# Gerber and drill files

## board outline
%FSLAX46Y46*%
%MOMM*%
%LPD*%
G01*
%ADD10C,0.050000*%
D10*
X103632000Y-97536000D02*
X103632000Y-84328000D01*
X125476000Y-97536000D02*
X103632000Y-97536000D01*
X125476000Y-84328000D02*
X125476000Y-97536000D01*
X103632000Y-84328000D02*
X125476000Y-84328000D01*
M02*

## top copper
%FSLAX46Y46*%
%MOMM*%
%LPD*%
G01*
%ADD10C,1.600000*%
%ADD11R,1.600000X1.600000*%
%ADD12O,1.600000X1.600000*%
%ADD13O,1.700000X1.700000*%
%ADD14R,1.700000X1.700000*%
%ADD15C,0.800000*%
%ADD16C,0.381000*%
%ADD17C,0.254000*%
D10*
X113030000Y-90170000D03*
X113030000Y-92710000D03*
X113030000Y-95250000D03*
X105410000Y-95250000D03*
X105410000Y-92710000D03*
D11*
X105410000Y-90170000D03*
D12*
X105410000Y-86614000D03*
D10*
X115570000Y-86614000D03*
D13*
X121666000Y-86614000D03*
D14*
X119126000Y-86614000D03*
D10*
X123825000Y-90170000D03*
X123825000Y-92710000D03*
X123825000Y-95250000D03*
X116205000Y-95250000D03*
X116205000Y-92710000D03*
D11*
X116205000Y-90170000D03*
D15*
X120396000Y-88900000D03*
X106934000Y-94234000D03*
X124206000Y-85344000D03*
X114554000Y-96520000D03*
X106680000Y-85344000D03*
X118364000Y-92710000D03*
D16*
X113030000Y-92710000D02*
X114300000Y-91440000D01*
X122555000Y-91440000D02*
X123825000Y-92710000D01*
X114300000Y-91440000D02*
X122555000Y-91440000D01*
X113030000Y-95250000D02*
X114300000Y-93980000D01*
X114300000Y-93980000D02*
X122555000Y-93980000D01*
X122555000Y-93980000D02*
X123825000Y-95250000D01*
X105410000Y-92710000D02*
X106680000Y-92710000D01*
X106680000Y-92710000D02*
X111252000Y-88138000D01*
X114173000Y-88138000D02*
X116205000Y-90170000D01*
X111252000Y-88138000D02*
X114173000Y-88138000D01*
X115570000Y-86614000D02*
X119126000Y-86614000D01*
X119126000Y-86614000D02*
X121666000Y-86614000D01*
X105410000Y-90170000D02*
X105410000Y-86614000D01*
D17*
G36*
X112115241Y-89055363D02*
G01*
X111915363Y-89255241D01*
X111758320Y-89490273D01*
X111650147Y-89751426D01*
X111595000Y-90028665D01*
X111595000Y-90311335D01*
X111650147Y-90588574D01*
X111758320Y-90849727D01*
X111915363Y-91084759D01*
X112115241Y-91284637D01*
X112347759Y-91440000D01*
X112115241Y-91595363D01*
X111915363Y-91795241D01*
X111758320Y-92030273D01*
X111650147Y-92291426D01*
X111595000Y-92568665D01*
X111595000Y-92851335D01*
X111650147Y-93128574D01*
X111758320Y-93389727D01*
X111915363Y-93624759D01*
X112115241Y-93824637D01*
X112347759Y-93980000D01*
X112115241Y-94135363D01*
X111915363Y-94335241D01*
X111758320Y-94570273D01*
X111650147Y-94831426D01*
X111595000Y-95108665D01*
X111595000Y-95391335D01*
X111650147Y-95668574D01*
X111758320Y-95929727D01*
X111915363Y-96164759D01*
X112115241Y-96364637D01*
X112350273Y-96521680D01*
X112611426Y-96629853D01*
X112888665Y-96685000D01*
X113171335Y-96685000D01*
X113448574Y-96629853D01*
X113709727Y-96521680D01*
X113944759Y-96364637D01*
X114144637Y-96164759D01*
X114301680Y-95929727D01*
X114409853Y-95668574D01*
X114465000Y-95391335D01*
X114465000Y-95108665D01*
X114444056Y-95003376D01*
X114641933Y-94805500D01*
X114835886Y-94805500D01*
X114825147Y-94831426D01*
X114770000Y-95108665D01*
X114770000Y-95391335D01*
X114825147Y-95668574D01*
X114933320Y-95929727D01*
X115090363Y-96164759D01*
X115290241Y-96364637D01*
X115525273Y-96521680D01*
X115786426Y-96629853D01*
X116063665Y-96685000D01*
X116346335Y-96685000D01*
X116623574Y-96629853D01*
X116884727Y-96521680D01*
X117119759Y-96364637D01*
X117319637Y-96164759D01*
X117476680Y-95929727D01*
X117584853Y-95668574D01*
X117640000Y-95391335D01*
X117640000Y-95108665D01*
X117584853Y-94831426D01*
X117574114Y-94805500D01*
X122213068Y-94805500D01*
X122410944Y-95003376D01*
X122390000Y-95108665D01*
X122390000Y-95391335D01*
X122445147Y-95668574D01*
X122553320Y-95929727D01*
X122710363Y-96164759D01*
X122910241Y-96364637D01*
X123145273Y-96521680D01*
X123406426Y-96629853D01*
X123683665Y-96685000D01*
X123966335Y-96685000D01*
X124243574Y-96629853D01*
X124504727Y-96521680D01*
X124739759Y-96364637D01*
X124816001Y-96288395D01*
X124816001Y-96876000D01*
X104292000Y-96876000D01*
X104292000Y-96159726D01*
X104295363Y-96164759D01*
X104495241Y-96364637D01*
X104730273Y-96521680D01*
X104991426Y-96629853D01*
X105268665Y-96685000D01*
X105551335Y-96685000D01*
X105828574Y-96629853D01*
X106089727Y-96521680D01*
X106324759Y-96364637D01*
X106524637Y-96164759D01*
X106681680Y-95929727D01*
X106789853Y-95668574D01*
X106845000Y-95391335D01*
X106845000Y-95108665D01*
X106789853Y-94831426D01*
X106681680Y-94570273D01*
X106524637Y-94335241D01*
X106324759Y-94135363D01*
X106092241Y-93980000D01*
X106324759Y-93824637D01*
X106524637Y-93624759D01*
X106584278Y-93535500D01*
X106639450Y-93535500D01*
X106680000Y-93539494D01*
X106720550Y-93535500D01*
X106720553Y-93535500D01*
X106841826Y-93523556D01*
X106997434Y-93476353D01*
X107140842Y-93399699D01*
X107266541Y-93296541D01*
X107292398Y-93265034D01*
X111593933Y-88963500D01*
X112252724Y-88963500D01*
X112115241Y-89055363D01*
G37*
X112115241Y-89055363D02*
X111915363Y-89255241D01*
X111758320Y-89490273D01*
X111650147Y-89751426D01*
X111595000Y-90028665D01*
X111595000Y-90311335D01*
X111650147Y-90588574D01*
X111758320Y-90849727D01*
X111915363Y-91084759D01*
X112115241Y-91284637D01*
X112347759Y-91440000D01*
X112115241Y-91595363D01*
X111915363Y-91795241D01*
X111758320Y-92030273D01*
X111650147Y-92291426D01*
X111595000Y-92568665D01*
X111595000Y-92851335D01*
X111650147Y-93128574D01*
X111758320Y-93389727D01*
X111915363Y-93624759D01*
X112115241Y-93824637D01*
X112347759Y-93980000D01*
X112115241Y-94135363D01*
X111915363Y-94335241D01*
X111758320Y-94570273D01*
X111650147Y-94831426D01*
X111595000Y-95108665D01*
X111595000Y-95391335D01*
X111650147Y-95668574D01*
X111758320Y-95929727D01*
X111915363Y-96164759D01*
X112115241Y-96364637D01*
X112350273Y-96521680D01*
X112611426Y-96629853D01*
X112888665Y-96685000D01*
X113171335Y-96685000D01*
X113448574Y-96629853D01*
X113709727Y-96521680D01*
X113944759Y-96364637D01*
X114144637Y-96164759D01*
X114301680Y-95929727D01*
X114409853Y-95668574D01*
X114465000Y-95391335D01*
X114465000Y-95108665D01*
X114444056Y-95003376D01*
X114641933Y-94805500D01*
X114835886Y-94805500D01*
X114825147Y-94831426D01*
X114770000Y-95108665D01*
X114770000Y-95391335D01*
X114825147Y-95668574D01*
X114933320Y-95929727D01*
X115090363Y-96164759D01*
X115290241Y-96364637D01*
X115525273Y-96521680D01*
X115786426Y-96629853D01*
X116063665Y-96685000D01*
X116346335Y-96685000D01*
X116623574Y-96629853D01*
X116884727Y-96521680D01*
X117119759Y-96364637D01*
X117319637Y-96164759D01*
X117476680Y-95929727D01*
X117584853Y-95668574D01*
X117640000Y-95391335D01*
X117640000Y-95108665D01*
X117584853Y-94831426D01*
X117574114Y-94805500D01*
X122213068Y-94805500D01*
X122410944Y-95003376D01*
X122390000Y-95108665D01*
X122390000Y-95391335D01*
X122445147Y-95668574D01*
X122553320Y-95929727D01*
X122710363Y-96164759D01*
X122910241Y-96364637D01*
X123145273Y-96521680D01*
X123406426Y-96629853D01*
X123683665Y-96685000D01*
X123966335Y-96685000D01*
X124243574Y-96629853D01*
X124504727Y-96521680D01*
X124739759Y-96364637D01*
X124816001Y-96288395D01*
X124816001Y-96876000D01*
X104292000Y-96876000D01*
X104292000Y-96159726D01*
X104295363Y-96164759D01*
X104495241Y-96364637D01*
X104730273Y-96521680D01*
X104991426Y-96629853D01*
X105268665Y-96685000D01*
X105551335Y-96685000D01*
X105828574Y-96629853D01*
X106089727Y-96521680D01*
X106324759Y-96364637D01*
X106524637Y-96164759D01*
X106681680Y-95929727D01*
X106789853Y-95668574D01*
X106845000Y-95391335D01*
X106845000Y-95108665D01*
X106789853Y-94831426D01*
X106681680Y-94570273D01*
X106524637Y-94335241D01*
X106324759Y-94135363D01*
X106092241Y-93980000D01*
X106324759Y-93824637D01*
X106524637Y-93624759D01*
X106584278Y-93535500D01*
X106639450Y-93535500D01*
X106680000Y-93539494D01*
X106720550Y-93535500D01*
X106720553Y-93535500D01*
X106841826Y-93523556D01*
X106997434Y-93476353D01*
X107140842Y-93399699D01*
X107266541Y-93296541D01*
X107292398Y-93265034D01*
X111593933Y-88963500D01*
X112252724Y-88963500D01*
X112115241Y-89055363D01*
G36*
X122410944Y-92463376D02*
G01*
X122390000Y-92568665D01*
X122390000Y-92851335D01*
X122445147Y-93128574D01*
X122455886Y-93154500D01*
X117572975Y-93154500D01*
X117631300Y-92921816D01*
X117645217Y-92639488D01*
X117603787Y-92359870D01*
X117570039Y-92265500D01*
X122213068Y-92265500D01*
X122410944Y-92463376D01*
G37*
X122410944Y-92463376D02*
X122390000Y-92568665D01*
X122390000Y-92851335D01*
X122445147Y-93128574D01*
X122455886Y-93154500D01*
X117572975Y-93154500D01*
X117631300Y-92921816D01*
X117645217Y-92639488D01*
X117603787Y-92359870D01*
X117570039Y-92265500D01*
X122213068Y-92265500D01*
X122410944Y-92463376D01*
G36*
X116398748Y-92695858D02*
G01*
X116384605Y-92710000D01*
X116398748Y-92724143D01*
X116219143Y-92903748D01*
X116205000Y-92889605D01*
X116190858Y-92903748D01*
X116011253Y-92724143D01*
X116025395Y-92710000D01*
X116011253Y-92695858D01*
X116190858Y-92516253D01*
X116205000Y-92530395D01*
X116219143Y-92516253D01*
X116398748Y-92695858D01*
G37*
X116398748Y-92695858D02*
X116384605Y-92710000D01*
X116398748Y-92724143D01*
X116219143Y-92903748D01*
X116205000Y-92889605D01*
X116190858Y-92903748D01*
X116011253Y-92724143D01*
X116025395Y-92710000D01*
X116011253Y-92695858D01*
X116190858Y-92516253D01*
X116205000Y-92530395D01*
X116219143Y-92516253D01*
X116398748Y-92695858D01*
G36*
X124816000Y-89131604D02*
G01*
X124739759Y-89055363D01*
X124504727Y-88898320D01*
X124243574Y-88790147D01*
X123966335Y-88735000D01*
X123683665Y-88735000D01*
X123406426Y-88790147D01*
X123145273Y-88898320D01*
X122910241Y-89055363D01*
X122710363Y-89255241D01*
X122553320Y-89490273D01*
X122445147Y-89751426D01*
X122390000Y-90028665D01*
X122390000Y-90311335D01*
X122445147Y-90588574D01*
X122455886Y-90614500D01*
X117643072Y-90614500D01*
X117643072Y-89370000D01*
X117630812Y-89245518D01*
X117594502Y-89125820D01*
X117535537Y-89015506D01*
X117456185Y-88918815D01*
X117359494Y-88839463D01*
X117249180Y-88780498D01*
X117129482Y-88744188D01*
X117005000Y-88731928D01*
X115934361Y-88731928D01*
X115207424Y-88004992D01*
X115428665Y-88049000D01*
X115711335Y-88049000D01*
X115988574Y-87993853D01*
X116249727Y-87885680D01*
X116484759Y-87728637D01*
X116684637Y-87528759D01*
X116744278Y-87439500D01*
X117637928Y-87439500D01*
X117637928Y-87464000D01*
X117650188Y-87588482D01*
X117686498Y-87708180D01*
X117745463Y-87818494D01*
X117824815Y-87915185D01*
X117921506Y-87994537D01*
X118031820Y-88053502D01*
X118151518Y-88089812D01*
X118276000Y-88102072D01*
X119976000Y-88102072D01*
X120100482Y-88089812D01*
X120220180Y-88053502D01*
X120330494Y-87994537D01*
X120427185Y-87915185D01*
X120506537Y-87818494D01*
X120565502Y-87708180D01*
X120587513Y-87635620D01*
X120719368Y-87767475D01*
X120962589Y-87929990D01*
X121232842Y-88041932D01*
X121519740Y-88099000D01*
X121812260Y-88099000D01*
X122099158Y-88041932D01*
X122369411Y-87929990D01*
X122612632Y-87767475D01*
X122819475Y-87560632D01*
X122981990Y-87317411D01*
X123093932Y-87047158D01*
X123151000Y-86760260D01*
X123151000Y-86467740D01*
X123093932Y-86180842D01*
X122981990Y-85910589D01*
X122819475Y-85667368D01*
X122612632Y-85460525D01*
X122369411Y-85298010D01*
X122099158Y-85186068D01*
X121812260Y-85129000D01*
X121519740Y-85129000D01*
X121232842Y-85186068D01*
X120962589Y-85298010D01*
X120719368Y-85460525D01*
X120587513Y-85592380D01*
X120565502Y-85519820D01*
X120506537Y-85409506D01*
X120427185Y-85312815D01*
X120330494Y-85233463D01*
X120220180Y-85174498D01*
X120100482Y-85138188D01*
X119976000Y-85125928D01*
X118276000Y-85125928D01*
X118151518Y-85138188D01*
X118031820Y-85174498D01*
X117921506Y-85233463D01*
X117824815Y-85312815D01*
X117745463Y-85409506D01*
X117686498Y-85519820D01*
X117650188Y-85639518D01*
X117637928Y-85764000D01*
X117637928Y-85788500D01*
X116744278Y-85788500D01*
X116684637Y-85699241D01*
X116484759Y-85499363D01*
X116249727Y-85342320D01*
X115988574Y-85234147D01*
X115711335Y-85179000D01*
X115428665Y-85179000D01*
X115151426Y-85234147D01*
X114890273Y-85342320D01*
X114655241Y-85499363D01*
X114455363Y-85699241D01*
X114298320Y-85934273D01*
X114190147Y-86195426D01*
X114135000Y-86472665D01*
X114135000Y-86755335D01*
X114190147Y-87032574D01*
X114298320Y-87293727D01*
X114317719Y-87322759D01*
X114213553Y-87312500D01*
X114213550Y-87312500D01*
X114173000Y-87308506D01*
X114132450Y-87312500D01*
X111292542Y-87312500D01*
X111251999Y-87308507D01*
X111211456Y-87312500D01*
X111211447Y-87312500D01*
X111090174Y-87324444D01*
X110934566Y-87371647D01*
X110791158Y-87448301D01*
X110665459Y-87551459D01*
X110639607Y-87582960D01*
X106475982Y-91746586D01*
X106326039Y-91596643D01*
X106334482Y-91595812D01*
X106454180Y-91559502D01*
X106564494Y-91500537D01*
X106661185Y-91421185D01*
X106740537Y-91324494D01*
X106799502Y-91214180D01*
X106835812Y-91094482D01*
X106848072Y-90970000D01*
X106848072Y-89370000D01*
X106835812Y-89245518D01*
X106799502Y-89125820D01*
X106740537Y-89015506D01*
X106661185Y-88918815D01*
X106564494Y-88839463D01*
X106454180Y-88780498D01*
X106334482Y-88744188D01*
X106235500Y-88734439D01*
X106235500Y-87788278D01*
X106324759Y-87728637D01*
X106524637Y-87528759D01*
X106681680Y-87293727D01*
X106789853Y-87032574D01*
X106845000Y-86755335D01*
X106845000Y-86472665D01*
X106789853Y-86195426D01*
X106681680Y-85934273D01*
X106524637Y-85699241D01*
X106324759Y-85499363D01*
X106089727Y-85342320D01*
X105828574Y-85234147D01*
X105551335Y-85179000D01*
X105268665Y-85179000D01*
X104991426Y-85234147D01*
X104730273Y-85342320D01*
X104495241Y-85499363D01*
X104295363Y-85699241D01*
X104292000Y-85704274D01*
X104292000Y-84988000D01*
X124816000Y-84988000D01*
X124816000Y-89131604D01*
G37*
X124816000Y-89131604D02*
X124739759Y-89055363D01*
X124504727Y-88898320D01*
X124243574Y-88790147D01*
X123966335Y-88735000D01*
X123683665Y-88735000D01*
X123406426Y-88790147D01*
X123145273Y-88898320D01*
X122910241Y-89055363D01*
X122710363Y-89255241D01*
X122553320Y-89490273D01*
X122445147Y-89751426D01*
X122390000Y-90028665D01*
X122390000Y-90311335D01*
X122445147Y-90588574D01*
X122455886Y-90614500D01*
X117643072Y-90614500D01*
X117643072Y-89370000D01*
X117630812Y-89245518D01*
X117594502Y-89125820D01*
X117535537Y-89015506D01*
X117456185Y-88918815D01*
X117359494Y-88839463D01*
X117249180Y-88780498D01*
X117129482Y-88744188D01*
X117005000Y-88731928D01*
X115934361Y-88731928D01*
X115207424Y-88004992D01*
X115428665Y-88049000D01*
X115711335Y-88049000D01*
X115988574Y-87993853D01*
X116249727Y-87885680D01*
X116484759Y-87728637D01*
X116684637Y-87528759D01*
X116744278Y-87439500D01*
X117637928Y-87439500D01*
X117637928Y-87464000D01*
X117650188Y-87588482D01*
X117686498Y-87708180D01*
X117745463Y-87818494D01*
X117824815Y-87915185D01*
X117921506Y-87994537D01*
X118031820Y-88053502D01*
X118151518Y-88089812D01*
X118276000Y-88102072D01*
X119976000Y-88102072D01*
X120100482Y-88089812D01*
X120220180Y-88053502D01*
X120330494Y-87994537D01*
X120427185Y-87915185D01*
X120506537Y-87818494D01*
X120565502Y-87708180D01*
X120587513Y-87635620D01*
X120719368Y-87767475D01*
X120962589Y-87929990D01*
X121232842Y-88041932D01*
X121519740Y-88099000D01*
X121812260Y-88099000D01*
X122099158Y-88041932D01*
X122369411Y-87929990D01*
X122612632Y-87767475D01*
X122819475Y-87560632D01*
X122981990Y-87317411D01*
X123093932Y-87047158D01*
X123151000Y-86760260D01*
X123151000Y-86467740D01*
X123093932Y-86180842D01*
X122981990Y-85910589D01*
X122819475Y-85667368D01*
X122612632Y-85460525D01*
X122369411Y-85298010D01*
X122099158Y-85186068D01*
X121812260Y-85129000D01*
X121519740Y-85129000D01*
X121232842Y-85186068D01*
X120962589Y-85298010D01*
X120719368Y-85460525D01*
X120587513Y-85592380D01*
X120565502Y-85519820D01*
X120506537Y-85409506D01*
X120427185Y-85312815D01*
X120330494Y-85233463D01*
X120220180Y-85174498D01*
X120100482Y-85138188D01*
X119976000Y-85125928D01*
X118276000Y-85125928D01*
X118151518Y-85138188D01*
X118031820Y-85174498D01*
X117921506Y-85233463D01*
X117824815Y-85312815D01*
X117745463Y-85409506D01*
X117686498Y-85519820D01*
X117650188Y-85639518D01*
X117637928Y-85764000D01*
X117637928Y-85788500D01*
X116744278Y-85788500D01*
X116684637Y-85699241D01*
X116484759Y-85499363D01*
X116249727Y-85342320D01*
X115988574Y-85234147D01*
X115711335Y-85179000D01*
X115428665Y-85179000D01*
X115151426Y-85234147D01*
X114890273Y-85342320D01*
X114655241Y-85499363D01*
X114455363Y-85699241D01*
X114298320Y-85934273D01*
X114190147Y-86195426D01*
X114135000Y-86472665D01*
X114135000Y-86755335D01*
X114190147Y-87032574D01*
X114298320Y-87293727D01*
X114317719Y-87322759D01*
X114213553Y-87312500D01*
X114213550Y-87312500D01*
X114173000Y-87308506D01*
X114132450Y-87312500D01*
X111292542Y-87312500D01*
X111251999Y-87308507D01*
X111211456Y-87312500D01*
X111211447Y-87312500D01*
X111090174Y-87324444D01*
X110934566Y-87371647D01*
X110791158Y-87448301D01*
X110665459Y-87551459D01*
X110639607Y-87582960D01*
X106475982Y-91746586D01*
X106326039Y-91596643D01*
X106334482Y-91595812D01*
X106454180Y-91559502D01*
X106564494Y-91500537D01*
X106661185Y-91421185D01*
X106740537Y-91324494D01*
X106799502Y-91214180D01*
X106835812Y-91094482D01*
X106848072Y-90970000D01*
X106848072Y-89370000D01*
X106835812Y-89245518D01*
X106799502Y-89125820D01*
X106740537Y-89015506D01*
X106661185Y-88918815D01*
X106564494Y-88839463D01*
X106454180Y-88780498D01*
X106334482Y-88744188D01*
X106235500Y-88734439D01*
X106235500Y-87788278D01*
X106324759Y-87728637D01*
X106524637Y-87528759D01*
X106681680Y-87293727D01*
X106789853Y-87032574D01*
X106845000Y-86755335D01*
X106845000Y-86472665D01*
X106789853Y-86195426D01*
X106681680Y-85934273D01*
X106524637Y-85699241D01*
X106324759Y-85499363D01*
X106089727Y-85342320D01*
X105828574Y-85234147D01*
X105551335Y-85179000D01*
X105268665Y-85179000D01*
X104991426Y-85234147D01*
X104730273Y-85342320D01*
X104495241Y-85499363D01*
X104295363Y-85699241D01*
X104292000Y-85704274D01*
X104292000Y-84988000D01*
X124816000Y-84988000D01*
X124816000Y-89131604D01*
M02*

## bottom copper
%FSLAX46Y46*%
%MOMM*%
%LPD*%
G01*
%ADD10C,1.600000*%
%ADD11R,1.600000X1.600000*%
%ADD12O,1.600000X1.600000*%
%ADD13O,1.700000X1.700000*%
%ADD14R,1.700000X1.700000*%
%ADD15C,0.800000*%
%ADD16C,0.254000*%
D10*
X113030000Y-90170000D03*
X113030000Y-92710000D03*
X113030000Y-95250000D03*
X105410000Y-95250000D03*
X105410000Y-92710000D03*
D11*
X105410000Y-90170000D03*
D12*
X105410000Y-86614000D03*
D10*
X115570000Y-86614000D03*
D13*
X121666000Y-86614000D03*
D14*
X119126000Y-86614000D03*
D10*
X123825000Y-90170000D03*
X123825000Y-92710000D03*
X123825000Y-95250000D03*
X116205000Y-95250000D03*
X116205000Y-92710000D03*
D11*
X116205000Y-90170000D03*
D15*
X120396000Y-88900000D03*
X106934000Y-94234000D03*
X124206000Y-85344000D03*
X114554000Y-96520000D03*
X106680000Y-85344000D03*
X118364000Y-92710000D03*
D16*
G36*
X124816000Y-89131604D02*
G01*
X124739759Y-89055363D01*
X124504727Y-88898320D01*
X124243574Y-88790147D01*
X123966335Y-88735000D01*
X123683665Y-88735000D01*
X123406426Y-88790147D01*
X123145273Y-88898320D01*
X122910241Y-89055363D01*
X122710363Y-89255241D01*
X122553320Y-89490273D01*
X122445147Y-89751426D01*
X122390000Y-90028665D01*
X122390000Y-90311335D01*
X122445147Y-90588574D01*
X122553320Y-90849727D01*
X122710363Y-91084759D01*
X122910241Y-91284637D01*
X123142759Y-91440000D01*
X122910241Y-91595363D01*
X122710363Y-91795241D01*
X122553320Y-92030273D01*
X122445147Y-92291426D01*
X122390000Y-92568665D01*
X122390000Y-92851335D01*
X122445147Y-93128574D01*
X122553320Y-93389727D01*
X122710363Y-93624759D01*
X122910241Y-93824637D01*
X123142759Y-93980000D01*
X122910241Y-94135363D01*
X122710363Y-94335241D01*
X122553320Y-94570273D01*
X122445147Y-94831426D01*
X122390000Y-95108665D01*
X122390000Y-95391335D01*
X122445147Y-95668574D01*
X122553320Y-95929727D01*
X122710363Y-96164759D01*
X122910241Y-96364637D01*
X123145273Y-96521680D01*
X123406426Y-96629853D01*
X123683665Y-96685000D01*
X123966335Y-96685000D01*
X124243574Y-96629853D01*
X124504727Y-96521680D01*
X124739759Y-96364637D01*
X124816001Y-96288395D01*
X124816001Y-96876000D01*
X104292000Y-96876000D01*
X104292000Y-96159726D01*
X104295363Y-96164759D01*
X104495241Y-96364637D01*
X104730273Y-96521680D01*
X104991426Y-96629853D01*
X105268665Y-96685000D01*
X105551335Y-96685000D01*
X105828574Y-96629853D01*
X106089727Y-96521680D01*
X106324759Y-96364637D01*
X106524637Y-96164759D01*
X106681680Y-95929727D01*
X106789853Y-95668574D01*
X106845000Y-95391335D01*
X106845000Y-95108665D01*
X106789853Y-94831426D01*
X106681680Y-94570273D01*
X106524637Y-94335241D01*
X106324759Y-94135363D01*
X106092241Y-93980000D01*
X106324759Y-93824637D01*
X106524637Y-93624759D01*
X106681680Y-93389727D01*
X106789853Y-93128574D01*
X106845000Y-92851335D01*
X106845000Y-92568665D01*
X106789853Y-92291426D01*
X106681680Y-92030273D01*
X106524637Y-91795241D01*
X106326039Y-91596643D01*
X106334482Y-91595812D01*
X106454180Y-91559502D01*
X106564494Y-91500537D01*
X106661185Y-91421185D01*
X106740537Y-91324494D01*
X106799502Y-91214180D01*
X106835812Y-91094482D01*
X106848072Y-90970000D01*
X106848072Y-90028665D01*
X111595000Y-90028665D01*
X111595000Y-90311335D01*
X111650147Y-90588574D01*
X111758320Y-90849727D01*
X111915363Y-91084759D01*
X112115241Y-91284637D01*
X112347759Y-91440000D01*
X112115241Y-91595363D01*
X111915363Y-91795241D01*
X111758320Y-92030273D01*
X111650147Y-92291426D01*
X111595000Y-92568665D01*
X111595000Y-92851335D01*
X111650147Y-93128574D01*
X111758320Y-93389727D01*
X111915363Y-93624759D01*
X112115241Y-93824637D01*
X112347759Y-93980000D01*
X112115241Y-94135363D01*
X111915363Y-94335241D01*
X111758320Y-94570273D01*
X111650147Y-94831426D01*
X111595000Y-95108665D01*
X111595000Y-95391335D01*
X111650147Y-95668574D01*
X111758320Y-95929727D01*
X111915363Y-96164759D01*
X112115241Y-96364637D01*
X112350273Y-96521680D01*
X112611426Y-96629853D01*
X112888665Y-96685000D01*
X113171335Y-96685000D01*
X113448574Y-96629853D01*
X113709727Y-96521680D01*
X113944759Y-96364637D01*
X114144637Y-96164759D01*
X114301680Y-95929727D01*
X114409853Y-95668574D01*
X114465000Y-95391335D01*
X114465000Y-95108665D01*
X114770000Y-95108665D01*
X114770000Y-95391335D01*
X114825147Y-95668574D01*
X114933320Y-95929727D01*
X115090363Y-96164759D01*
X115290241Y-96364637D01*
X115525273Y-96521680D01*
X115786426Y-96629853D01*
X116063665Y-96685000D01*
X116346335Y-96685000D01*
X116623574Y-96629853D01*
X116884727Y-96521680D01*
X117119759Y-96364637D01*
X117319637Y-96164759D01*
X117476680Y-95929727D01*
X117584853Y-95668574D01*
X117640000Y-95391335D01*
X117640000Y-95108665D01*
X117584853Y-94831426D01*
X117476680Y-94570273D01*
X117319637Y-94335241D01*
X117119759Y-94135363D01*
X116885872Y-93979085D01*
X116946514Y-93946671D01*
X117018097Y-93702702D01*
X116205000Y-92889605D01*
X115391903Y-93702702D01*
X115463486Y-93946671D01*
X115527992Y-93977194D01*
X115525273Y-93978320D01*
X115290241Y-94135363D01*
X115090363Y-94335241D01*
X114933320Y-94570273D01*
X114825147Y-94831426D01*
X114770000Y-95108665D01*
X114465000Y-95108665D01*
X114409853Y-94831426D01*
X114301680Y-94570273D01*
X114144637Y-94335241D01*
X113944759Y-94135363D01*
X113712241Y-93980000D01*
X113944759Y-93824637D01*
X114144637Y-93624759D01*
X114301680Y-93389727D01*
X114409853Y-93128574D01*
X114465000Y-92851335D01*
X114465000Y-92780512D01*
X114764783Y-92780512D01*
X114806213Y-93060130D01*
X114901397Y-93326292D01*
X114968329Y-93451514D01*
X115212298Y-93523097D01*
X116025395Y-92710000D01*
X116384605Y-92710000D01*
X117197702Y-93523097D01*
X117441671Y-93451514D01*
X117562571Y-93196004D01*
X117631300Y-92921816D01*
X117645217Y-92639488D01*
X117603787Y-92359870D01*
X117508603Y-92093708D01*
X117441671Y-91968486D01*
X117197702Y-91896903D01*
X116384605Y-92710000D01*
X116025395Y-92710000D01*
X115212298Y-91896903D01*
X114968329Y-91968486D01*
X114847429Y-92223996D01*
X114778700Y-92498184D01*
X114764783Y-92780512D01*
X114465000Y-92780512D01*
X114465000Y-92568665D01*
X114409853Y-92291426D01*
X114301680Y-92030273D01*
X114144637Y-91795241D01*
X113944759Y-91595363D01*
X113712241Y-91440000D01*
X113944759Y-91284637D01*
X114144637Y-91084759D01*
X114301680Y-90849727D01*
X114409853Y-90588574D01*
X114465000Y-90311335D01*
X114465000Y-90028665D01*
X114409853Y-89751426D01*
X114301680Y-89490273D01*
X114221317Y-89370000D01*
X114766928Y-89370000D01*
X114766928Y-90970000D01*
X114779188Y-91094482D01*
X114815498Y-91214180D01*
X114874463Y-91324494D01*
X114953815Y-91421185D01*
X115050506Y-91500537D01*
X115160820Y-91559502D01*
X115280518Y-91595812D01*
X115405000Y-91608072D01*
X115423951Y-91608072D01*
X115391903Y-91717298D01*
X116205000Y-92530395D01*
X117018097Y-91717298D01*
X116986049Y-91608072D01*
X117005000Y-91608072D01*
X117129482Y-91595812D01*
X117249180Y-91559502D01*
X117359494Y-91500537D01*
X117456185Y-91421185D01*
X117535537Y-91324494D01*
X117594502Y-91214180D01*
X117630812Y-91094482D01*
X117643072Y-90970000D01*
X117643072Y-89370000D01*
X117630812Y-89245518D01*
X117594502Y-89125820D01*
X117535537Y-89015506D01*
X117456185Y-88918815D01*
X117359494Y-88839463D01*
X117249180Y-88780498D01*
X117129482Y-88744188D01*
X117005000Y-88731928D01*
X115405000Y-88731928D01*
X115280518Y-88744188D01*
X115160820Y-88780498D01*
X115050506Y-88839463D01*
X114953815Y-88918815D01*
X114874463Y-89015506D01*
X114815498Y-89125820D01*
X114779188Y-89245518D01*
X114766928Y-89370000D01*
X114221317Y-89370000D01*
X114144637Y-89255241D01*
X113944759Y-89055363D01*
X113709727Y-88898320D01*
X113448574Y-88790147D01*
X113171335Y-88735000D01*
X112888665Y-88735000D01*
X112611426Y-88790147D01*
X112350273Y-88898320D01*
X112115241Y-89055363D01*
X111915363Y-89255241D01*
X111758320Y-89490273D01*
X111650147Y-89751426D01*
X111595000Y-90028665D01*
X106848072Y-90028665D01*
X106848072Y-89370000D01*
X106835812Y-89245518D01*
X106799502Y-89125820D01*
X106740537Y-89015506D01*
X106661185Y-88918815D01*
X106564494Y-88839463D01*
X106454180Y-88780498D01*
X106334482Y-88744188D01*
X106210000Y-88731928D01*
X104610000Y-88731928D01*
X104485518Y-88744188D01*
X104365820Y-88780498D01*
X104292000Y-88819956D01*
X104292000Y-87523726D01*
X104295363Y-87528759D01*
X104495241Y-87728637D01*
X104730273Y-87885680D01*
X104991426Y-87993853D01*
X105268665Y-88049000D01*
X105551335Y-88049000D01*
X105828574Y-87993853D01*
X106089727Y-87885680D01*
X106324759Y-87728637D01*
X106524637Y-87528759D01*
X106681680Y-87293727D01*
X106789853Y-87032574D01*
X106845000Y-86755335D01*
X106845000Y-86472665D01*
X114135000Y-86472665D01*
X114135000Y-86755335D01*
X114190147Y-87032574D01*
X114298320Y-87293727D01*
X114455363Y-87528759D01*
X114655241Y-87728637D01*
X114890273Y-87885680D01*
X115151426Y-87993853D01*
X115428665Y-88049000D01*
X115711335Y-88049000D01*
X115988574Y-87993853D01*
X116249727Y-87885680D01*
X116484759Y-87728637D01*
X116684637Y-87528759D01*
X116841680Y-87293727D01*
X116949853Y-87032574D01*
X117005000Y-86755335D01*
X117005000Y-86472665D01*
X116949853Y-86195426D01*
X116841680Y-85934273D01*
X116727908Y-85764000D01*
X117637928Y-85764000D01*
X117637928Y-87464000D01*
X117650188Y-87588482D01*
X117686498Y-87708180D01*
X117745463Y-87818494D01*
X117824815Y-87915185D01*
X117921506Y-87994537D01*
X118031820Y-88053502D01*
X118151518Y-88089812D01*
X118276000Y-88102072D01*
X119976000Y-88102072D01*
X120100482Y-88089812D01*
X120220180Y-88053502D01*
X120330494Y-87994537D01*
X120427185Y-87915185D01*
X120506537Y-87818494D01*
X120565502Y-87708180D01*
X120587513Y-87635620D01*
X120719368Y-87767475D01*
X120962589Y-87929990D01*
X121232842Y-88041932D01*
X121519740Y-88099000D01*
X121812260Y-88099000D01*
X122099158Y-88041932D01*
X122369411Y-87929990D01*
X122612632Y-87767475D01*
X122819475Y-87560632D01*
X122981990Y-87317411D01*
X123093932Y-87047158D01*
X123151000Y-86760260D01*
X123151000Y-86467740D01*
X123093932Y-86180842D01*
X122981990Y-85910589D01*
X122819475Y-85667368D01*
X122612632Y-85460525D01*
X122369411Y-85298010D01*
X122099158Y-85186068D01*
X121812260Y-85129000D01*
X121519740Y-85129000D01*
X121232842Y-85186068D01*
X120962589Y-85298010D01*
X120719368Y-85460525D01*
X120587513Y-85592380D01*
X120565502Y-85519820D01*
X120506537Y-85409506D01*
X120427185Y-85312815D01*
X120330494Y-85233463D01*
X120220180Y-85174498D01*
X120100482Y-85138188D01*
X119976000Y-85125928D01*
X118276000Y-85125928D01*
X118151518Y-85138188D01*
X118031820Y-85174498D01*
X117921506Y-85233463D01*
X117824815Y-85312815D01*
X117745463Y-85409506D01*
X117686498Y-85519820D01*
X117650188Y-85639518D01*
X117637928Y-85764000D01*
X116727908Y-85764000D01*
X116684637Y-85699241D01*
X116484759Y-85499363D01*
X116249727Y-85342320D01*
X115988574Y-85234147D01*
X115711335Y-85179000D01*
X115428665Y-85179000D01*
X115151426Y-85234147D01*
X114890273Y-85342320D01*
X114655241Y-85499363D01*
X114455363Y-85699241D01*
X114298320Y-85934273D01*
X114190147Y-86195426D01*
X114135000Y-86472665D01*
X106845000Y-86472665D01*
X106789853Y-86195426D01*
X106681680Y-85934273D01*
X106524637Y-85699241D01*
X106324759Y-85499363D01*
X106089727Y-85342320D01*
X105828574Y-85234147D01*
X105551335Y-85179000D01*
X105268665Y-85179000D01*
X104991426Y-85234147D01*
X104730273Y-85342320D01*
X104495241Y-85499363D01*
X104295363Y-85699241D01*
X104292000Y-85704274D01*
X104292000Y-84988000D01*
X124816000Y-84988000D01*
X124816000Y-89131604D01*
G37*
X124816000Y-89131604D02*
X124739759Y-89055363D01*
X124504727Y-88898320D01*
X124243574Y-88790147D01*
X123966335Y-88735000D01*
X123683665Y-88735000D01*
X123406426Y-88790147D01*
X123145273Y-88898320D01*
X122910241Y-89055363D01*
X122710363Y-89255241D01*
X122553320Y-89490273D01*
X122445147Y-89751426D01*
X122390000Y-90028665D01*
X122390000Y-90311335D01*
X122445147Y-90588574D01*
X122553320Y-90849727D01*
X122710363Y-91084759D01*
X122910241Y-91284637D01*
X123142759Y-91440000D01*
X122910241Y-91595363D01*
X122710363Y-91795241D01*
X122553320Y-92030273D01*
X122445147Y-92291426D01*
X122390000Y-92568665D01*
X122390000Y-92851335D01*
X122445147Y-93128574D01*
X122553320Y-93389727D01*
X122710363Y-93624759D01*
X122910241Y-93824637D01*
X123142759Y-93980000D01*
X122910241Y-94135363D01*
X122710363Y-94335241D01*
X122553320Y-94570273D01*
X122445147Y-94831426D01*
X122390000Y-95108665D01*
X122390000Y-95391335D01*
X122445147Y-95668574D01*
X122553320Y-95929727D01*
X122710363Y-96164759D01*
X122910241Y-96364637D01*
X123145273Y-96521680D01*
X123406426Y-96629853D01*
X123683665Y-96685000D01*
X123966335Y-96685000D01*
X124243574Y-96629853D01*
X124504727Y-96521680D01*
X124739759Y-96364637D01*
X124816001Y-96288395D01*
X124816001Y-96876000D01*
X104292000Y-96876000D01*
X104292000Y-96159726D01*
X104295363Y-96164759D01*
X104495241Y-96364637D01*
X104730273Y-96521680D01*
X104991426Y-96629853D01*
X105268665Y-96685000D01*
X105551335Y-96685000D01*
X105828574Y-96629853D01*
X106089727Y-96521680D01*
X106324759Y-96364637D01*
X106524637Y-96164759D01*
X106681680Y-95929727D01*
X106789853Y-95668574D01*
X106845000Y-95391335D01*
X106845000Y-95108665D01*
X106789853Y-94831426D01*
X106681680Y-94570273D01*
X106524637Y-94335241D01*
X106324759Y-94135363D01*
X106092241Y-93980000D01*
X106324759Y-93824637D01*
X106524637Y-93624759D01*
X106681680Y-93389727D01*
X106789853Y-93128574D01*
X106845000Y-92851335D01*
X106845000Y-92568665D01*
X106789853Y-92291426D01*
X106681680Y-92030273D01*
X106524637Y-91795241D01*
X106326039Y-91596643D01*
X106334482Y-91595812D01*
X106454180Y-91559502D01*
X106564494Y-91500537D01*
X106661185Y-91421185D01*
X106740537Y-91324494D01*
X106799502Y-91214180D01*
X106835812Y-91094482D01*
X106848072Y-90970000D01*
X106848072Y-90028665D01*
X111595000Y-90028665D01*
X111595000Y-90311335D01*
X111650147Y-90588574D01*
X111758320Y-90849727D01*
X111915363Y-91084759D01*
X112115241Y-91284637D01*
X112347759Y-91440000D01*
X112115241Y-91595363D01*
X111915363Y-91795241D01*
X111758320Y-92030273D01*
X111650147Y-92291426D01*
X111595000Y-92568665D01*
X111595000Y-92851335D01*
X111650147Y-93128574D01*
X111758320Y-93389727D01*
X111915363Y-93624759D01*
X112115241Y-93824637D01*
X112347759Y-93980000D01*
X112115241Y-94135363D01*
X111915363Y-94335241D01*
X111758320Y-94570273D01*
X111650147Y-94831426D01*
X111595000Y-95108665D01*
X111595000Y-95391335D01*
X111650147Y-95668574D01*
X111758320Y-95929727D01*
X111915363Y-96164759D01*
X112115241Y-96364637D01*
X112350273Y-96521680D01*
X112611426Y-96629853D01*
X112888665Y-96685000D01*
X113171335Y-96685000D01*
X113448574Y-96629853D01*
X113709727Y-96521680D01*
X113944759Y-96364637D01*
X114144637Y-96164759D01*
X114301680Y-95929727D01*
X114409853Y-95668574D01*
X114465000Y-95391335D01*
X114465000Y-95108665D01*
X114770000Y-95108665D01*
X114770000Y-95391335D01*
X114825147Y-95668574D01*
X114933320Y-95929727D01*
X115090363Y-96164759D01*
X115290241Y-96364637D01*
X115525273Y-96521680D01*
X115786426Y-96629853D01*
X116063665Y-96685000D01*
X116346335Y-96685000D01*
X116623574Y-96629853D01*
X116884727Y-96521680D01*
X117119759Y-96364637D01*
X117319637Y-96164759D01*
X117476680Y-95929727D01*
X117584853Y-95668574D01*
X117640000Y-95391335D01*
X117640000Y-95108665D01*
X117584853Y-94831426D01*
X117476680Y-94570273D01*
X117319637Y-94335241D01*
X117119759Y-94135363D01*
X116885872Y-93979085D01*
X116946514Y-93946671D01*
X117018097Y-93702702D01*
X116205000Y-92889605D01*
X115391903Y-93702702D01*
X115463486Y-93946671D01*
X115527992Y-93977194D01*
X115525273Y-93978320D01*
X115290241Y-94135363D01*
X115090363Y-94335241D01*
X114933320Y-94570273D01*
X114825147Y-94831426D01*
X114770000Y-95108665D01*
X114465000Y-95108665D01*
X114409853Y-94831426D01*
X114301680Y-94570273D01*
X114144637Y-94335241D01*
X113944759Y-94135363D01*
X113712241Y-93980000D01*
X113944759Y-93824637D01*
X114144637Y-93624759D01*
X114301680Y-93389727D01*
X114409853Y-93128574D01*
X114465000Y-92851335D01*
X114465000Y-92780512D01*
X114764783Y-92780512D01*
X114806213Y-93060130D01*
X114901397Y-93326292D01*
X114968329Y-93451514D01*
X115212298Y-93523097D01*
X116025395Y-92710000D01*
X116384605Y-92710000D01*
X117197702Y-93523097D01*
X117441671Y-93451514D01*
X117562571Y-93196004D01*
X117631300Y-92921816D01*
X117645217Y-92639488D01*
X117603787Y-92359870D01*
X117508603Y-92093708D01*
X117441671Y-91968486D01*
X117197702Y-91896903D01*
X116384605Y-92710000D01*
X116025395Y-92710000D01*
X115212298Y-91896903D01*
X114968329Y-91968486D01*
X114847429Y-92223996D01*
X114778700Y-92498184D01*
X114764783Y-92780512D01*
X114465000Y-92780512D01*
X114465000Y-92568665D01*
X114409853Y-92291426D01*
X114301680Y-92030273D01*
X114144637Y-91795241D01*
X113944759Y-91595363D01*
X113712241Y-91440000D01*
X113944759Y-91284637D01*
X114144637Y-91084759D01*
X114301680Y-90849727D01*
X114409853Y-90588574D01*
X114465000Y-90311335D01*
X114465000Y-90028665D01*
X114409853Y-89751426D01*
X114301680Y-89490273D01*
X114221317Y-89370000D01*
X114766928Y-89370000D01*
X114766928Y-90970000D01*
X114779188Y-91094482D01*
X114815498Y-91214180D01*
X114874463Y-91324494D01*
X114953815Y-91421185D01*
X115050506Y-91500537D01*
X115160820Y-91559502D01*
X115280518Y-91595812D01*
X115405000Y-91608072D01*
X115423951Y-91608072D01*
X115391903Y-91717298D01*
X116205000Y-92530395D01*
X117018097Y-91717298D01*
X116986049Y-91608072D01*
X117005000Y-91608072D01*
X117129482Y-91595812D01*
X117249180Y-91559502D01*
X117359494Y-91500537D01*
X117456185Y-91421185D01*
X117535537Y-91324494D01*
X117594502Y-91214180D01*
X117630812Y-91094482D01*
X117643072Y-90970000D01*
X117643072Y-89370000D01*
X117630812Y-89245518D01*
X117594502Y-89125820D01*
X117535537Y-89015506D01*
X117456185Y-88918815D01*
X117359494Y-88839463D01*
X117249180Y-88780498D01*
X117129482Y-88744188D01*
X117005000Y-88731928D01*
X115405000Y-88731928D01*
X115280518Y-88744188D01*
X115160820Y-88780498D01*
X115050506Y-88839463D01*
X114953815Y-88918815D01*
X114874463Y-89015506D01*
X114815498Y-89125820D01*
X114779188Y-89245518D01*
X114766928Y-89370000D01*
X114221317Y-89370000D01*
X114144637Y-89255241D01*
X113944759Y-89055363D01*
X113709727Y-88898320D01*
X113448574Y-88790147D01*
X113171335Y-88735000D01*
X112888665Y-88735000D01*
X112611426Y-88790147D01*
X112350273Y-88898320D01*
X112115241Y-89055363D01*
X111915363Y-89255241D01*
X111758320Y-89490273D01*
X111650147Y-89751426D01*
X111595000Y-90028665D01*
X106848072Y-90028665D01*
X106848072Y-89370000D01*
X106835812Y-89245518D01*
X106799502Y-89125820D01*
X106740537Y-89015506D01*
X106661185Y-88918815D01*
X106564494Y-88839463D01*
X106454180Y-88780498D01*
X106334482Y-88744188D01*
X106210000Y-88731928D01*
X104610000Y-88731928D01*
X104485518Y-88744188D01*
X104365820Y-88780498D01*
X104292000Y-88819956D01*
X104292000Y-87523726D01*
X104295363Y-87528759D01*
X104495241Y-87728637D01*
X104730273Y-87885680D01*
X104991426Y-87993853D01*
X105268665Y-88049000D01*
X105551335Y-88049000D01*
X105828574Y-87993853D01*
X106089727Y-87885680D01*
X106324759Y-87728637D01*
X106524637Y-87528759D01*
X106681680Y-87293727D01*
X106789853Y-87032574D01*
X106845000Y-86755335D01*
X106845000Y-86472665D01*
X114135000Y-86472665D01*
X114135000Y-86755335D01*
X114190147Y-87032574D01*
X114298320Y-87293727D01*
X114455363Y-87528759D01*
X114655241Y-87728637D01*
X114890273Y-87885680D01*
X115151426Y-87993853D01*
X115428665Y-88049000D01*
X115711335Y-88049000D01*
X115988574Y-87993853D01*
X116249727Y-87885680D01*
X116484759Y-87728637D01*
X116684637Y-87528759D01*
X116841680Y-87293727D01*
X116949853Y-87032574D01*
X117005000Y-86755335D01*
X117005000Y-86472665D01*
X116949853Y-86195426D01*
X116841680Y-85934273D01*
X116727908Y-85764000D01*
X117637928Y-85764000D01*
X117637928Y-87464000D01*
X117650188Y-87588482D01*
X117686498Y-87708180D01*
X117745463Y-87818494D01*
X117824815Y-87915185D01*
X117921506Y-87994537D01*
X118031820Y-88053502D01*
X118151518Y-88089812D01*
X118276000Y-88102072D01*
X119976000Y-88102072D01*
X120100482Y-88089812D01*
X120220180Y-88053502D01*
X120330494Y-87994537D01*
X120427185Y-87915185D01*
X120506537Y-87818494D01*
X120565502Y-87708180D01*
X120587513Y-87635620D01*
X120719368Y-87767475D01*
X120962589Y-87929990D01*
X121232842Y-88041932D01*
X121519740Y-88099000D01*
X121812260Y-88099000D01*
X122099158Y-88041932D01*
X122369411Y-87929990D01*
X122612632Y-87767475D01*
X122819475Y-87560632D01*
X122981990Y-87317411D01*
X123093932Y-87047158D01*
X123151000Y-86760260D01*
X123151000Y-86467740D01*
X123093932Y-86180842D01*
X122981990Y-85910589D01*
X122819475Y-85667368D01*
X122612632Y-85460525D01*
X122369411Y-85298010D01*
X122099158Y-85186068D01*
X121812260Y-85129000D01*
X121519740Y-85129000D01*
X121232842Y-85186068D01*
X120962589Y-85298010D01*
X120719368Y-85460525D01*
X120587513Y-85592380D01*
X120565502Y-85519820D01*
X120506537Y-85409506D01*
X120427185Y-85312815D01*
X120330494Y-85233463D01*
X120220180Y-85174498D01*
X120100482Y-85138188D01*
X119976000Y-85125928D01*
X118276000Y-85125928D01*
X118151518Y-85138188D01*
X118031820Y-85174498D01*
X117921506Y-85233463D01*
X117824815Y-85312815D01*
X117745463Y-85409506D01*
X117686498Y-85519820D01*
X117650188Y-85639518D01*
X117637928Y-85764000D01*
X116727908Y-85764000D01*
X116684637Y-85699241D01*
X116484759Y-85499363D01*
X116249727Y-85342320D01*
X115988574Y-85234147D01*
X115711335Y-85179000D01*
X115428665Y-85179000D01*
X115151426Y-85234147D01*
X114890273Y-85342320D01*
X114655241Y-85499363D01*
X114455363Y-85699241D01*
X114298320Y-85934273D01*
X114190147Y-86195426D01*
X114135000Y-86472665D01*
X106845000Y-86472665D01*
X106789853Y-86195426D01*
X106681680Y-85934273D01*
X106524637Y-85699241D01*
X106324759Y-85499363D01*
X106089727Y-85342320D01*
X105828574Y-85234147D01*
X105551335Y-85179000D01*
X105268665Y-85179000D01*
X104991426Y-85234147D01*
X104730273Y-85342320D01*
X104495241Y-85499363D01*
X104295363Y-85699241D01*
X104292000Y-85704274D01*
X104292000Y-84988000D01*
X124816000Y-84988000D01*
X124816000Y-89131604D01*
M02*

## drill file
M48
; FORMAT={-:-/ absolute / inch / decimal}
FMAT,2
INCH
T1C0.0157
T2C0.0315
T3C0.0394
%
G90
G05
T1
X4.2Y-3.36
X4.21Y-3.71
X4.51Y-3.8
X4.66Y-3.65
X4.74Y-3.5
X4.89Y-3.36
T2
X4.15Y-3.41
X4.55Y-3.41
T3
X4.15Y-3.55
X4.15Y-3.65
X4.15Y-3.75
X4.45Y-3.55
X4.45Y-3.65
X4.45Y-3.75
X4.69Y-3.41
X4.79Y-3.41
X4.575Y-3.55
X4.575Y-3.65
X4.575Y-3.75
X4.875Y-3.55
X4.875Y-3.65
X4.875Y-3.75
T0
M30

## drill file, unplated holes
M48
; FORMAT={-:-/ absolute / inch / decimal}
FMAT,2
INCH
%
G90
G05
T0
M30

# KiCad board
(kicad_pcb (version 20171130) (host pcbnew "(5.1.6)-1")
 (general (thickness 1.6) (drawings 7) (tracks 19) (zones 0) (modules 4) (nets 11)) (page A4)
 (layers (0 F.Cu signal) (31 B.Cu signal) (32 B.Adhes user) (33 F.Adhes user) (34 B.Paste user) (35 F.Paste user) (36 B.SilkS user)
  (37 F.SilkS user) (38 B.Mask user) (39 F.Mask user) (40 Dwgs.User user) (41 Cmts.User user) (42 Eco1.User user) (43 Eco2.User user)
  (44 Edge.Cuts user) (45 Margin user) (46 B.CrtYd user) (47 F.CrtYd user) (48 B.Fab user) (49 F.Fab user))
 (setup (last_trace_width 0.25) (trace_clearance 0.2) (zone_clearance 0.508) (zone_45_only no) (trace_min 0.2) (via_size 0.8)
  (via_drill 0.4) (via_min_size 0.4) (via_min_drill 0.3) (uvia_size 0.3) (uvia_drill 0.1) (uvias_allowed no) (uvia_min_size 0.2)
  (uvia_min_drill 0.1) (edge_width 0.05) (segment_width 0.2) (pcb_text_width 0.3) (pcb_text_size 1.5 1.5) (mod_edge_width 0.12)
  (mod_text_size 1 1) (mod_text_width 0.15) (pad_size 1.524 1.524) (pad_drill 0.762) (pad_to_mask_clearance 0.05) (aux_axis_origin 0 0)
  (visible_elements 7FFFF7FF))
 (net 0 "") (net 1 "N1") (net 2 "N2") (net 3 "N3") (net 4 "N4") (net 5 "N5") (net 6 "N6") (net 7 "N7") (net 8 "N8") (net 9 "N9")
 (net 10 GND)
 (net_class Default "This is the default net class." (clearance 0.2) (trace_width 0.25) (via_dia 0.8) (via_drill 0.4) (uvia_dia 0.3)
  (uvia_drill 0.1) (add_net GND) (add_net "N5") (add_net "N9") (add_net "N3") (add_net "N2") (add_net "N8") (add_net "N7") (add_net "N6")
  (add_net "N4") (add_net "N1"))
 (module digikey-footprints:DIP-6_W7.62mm (layer F.Cu) (at 105.41 90.17)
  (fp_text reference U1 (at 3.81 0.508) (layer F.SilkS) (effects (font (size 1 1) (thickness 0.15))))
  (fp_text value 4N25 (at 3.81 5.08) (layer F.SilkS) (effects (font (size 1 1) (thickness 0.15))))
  (pad 6 thru_hole circle (at 7.62 0) (size 1.6 1.6) (drill 1) (layers *.Cu *.Mask) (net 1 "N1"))
  (pad 5 thru_hole circle (at 7.62 2.54) (size 1.6 1.6) (drill 1) (layers *.Cu *.Mask) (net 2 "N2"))
  (pad 4 thru_hole circle (at 7.62 5.08) (size 1.6 1.6) (drill 1) (layers *.Cu *.Mask) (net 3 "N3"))
  (pad 3 thru_hole circle (at 0 5.08) (size 1.6 1.6) (drill 1) (layers *.Cu *.Mask) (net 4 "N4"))
  (pad 2 thru_hole circle (at 0 2.54) (size 1.6 1.6) (drill 1) (layers *.Cu *.Mask) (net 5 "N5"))
  (pad 1 thru_hole rect (at 0 0) (size 1.6 1.6) (drill 1) (layers *.Cu *.Mask) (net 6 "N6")))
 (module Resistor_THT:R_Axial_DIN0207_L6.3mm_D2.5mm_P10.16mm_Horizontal (layer F.Cu) (at 115.57 86.614 180)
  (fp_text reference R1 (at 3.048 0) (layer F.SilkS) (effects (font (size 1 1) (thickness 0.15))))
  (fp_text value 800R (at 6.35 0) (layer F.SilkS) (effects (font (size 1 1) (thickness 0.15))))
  (pad 2 thru_hole oval (at 10.16 0 180) (size 1.6 1.6) (drill 0.8) (layers *.Cu *.Mask) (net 6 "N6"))
  (pad 1 thru_hole circle (at 0 0 180) (size 1.6 1.6) (drill 0.8) (layers *.Cu *.Mask) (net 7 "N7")))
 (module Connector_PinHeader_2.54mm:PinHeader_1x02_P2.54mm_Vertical (layer F.Cu) (at 119.126 86.614 90)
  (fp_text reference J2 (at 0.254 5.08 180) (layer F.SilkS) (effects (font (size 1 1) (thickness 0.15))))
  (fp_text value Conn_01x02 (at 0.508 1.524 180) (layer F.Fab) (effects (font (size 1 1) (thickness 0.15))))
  (pad 2 thru_hole oval (at 0 2.54 90) (size 1.7 1.7) (drill 1) (layers *.Cu *.Mask) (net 7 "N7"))
  (pad 1 thru_hole rect (at 0 0 90) (size 1.7 1.7) (drill 1) (layers *.Cu *.Mask) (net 7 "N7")))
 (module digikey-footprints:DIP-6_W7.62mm (layer F.Cu) (at 116.205 90.17)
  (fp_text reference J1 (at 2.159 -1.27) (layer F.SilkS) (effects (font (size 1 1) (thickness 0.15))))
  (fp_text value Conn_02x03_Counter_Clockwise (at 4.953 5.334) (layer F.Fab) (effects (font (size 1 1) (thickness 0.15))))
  (pad 6 thru_hole circle (at 7.62 0) (size 1.6 1.6) (drill 1) (layers *.Cu *.Mask) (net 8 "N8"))
  (pad 5 thru_hole circle (at 7.62 2.54) (size 1.6 1.6) (drill 1) (layers *.Cu *.Mask) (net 2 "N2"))
  (pad 4 thru_hole circle (at 7.62 5.08) (size 1.6 1.6) (drill 1) (layers *.Cu *.Mask) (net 3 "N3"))
  (pad 3 thru_hole circle (at 0 5.08) (size 1.6 1.6) (drill 1) (layers *.Cu *.Mask) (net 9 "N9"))
  (pad 2 thru_hole circle (at 0 2.54) (size 1.6 1.6) (drill 1) (layers *.Cu *.Mask) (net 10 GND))
  (pad 1 thru_hole rect (at 0 0) (size 1.6 1.6) (drill 1) (layers *.Cu *.Mask) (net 5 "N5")))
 (gr_line (start 103.632 97.536) (end 103.632 84.328) (layer Edge.Cuts) (width 0.05))
 (gr_line (start 125.476 97.536) (end 103.632 97.536) (layer Edge.Cuts) (width 0.05))
 (gr_line (start 125.476 84.328) (end 125.476 97.536) (layer Edge.Cuts) (width 0.05))
 (gr_line (start 103.632 84.328) (end 125.476 84.328) (layer Edge.Cuts) (width 0.05))
 (segment (start 113.03 92.71) (end 114.3 91.44) (width 0.381) (layer F.Cu) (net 2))
 (segment (start 122.555 91.44) (end 123.825 92.71) (width 0.381) (layer F.Cu) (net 2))
 (segment (start 114.3 91.44) (end 122.555 91.44) (width 0.381) (layer F.Cu) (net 2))
 (segment (start 113.03 95.25) (end 114.3 93.98) (width 0.381) (layer F.Cu) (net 3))
 (segment (start 114.3 93.98) (end 122.555 93.98) (width 0.381) (layer F.Cu) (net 3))
 (segment (start 122.555 93.98) (end 123.825 95.25) (width 0.381) (layer F.Cu) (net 3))
 (via (at 120.396 88.9) (size 0.8) (drill 0.4) (layers F.Cu B.Cu) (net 10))
 (via (at 106.934 94.234) (size 0.8) (drill 0.4) (layers F.Cu B.Cu) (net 10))
 (via (at 124.206 85.344) (size 0.8) (drill 0.4) (layers F.Cu B.Cu) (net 10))
 (via (at 114.554 96.52) (size 0.8) (drill 0.4) (layers F.Cu B.Cu) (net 10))
 (via (at 106.68 85.344) (size 0.8) (drill 0.4) (layers F.Cu B.Cu) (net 10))
 (via (at 118.364 92.71) (size 0.8) (drill 0.4) (layers F.Cu B.Cu) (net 10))
 (segment (start 105.41 92.71) (end 106.68 92.71) (width 0.381) (layer F.Cu) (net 5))
 (segment (start 106.68 92.71) (end 111.252 88.138) (width 0.381) (layer F.Cu) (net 5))
 (segment (start 114.173 88.138) (end 116.205 90.17) (width 0.381) (layer F.Cu) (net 5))
 (segment (start 111.252 88.138) (end 114.173 88.138) (width 0.381) (layer F.Cu) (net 5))
 (segment (start 115.57 86.614) (end 119.126 86.614) (width 0.381) (layer F.Cu) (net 7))
 (segment (start 119.126 86.614) (end 121.666 86.614) (width 0.381) (layer F.Cu) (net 7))
 (segment (start 105.41 90.17) (end 105.41 86.614) (width 0.381) (layer F.Cu) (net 6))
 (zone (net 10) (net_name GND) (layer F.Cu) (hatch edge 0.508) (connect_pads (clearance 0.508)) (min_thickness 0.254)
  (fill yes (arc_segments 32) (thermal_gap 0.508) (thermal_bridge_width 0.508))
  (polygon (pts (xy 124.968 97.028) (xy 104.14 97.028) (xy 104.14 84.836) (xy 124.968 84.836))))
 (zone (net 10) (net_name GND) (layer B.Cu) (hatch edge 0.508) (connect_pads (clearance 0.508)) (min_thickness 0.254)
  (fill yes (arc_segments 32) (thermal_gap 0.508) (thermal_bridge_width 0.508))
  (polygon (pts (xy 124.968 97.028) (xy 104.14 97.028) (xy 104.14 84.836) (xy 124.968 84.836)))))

